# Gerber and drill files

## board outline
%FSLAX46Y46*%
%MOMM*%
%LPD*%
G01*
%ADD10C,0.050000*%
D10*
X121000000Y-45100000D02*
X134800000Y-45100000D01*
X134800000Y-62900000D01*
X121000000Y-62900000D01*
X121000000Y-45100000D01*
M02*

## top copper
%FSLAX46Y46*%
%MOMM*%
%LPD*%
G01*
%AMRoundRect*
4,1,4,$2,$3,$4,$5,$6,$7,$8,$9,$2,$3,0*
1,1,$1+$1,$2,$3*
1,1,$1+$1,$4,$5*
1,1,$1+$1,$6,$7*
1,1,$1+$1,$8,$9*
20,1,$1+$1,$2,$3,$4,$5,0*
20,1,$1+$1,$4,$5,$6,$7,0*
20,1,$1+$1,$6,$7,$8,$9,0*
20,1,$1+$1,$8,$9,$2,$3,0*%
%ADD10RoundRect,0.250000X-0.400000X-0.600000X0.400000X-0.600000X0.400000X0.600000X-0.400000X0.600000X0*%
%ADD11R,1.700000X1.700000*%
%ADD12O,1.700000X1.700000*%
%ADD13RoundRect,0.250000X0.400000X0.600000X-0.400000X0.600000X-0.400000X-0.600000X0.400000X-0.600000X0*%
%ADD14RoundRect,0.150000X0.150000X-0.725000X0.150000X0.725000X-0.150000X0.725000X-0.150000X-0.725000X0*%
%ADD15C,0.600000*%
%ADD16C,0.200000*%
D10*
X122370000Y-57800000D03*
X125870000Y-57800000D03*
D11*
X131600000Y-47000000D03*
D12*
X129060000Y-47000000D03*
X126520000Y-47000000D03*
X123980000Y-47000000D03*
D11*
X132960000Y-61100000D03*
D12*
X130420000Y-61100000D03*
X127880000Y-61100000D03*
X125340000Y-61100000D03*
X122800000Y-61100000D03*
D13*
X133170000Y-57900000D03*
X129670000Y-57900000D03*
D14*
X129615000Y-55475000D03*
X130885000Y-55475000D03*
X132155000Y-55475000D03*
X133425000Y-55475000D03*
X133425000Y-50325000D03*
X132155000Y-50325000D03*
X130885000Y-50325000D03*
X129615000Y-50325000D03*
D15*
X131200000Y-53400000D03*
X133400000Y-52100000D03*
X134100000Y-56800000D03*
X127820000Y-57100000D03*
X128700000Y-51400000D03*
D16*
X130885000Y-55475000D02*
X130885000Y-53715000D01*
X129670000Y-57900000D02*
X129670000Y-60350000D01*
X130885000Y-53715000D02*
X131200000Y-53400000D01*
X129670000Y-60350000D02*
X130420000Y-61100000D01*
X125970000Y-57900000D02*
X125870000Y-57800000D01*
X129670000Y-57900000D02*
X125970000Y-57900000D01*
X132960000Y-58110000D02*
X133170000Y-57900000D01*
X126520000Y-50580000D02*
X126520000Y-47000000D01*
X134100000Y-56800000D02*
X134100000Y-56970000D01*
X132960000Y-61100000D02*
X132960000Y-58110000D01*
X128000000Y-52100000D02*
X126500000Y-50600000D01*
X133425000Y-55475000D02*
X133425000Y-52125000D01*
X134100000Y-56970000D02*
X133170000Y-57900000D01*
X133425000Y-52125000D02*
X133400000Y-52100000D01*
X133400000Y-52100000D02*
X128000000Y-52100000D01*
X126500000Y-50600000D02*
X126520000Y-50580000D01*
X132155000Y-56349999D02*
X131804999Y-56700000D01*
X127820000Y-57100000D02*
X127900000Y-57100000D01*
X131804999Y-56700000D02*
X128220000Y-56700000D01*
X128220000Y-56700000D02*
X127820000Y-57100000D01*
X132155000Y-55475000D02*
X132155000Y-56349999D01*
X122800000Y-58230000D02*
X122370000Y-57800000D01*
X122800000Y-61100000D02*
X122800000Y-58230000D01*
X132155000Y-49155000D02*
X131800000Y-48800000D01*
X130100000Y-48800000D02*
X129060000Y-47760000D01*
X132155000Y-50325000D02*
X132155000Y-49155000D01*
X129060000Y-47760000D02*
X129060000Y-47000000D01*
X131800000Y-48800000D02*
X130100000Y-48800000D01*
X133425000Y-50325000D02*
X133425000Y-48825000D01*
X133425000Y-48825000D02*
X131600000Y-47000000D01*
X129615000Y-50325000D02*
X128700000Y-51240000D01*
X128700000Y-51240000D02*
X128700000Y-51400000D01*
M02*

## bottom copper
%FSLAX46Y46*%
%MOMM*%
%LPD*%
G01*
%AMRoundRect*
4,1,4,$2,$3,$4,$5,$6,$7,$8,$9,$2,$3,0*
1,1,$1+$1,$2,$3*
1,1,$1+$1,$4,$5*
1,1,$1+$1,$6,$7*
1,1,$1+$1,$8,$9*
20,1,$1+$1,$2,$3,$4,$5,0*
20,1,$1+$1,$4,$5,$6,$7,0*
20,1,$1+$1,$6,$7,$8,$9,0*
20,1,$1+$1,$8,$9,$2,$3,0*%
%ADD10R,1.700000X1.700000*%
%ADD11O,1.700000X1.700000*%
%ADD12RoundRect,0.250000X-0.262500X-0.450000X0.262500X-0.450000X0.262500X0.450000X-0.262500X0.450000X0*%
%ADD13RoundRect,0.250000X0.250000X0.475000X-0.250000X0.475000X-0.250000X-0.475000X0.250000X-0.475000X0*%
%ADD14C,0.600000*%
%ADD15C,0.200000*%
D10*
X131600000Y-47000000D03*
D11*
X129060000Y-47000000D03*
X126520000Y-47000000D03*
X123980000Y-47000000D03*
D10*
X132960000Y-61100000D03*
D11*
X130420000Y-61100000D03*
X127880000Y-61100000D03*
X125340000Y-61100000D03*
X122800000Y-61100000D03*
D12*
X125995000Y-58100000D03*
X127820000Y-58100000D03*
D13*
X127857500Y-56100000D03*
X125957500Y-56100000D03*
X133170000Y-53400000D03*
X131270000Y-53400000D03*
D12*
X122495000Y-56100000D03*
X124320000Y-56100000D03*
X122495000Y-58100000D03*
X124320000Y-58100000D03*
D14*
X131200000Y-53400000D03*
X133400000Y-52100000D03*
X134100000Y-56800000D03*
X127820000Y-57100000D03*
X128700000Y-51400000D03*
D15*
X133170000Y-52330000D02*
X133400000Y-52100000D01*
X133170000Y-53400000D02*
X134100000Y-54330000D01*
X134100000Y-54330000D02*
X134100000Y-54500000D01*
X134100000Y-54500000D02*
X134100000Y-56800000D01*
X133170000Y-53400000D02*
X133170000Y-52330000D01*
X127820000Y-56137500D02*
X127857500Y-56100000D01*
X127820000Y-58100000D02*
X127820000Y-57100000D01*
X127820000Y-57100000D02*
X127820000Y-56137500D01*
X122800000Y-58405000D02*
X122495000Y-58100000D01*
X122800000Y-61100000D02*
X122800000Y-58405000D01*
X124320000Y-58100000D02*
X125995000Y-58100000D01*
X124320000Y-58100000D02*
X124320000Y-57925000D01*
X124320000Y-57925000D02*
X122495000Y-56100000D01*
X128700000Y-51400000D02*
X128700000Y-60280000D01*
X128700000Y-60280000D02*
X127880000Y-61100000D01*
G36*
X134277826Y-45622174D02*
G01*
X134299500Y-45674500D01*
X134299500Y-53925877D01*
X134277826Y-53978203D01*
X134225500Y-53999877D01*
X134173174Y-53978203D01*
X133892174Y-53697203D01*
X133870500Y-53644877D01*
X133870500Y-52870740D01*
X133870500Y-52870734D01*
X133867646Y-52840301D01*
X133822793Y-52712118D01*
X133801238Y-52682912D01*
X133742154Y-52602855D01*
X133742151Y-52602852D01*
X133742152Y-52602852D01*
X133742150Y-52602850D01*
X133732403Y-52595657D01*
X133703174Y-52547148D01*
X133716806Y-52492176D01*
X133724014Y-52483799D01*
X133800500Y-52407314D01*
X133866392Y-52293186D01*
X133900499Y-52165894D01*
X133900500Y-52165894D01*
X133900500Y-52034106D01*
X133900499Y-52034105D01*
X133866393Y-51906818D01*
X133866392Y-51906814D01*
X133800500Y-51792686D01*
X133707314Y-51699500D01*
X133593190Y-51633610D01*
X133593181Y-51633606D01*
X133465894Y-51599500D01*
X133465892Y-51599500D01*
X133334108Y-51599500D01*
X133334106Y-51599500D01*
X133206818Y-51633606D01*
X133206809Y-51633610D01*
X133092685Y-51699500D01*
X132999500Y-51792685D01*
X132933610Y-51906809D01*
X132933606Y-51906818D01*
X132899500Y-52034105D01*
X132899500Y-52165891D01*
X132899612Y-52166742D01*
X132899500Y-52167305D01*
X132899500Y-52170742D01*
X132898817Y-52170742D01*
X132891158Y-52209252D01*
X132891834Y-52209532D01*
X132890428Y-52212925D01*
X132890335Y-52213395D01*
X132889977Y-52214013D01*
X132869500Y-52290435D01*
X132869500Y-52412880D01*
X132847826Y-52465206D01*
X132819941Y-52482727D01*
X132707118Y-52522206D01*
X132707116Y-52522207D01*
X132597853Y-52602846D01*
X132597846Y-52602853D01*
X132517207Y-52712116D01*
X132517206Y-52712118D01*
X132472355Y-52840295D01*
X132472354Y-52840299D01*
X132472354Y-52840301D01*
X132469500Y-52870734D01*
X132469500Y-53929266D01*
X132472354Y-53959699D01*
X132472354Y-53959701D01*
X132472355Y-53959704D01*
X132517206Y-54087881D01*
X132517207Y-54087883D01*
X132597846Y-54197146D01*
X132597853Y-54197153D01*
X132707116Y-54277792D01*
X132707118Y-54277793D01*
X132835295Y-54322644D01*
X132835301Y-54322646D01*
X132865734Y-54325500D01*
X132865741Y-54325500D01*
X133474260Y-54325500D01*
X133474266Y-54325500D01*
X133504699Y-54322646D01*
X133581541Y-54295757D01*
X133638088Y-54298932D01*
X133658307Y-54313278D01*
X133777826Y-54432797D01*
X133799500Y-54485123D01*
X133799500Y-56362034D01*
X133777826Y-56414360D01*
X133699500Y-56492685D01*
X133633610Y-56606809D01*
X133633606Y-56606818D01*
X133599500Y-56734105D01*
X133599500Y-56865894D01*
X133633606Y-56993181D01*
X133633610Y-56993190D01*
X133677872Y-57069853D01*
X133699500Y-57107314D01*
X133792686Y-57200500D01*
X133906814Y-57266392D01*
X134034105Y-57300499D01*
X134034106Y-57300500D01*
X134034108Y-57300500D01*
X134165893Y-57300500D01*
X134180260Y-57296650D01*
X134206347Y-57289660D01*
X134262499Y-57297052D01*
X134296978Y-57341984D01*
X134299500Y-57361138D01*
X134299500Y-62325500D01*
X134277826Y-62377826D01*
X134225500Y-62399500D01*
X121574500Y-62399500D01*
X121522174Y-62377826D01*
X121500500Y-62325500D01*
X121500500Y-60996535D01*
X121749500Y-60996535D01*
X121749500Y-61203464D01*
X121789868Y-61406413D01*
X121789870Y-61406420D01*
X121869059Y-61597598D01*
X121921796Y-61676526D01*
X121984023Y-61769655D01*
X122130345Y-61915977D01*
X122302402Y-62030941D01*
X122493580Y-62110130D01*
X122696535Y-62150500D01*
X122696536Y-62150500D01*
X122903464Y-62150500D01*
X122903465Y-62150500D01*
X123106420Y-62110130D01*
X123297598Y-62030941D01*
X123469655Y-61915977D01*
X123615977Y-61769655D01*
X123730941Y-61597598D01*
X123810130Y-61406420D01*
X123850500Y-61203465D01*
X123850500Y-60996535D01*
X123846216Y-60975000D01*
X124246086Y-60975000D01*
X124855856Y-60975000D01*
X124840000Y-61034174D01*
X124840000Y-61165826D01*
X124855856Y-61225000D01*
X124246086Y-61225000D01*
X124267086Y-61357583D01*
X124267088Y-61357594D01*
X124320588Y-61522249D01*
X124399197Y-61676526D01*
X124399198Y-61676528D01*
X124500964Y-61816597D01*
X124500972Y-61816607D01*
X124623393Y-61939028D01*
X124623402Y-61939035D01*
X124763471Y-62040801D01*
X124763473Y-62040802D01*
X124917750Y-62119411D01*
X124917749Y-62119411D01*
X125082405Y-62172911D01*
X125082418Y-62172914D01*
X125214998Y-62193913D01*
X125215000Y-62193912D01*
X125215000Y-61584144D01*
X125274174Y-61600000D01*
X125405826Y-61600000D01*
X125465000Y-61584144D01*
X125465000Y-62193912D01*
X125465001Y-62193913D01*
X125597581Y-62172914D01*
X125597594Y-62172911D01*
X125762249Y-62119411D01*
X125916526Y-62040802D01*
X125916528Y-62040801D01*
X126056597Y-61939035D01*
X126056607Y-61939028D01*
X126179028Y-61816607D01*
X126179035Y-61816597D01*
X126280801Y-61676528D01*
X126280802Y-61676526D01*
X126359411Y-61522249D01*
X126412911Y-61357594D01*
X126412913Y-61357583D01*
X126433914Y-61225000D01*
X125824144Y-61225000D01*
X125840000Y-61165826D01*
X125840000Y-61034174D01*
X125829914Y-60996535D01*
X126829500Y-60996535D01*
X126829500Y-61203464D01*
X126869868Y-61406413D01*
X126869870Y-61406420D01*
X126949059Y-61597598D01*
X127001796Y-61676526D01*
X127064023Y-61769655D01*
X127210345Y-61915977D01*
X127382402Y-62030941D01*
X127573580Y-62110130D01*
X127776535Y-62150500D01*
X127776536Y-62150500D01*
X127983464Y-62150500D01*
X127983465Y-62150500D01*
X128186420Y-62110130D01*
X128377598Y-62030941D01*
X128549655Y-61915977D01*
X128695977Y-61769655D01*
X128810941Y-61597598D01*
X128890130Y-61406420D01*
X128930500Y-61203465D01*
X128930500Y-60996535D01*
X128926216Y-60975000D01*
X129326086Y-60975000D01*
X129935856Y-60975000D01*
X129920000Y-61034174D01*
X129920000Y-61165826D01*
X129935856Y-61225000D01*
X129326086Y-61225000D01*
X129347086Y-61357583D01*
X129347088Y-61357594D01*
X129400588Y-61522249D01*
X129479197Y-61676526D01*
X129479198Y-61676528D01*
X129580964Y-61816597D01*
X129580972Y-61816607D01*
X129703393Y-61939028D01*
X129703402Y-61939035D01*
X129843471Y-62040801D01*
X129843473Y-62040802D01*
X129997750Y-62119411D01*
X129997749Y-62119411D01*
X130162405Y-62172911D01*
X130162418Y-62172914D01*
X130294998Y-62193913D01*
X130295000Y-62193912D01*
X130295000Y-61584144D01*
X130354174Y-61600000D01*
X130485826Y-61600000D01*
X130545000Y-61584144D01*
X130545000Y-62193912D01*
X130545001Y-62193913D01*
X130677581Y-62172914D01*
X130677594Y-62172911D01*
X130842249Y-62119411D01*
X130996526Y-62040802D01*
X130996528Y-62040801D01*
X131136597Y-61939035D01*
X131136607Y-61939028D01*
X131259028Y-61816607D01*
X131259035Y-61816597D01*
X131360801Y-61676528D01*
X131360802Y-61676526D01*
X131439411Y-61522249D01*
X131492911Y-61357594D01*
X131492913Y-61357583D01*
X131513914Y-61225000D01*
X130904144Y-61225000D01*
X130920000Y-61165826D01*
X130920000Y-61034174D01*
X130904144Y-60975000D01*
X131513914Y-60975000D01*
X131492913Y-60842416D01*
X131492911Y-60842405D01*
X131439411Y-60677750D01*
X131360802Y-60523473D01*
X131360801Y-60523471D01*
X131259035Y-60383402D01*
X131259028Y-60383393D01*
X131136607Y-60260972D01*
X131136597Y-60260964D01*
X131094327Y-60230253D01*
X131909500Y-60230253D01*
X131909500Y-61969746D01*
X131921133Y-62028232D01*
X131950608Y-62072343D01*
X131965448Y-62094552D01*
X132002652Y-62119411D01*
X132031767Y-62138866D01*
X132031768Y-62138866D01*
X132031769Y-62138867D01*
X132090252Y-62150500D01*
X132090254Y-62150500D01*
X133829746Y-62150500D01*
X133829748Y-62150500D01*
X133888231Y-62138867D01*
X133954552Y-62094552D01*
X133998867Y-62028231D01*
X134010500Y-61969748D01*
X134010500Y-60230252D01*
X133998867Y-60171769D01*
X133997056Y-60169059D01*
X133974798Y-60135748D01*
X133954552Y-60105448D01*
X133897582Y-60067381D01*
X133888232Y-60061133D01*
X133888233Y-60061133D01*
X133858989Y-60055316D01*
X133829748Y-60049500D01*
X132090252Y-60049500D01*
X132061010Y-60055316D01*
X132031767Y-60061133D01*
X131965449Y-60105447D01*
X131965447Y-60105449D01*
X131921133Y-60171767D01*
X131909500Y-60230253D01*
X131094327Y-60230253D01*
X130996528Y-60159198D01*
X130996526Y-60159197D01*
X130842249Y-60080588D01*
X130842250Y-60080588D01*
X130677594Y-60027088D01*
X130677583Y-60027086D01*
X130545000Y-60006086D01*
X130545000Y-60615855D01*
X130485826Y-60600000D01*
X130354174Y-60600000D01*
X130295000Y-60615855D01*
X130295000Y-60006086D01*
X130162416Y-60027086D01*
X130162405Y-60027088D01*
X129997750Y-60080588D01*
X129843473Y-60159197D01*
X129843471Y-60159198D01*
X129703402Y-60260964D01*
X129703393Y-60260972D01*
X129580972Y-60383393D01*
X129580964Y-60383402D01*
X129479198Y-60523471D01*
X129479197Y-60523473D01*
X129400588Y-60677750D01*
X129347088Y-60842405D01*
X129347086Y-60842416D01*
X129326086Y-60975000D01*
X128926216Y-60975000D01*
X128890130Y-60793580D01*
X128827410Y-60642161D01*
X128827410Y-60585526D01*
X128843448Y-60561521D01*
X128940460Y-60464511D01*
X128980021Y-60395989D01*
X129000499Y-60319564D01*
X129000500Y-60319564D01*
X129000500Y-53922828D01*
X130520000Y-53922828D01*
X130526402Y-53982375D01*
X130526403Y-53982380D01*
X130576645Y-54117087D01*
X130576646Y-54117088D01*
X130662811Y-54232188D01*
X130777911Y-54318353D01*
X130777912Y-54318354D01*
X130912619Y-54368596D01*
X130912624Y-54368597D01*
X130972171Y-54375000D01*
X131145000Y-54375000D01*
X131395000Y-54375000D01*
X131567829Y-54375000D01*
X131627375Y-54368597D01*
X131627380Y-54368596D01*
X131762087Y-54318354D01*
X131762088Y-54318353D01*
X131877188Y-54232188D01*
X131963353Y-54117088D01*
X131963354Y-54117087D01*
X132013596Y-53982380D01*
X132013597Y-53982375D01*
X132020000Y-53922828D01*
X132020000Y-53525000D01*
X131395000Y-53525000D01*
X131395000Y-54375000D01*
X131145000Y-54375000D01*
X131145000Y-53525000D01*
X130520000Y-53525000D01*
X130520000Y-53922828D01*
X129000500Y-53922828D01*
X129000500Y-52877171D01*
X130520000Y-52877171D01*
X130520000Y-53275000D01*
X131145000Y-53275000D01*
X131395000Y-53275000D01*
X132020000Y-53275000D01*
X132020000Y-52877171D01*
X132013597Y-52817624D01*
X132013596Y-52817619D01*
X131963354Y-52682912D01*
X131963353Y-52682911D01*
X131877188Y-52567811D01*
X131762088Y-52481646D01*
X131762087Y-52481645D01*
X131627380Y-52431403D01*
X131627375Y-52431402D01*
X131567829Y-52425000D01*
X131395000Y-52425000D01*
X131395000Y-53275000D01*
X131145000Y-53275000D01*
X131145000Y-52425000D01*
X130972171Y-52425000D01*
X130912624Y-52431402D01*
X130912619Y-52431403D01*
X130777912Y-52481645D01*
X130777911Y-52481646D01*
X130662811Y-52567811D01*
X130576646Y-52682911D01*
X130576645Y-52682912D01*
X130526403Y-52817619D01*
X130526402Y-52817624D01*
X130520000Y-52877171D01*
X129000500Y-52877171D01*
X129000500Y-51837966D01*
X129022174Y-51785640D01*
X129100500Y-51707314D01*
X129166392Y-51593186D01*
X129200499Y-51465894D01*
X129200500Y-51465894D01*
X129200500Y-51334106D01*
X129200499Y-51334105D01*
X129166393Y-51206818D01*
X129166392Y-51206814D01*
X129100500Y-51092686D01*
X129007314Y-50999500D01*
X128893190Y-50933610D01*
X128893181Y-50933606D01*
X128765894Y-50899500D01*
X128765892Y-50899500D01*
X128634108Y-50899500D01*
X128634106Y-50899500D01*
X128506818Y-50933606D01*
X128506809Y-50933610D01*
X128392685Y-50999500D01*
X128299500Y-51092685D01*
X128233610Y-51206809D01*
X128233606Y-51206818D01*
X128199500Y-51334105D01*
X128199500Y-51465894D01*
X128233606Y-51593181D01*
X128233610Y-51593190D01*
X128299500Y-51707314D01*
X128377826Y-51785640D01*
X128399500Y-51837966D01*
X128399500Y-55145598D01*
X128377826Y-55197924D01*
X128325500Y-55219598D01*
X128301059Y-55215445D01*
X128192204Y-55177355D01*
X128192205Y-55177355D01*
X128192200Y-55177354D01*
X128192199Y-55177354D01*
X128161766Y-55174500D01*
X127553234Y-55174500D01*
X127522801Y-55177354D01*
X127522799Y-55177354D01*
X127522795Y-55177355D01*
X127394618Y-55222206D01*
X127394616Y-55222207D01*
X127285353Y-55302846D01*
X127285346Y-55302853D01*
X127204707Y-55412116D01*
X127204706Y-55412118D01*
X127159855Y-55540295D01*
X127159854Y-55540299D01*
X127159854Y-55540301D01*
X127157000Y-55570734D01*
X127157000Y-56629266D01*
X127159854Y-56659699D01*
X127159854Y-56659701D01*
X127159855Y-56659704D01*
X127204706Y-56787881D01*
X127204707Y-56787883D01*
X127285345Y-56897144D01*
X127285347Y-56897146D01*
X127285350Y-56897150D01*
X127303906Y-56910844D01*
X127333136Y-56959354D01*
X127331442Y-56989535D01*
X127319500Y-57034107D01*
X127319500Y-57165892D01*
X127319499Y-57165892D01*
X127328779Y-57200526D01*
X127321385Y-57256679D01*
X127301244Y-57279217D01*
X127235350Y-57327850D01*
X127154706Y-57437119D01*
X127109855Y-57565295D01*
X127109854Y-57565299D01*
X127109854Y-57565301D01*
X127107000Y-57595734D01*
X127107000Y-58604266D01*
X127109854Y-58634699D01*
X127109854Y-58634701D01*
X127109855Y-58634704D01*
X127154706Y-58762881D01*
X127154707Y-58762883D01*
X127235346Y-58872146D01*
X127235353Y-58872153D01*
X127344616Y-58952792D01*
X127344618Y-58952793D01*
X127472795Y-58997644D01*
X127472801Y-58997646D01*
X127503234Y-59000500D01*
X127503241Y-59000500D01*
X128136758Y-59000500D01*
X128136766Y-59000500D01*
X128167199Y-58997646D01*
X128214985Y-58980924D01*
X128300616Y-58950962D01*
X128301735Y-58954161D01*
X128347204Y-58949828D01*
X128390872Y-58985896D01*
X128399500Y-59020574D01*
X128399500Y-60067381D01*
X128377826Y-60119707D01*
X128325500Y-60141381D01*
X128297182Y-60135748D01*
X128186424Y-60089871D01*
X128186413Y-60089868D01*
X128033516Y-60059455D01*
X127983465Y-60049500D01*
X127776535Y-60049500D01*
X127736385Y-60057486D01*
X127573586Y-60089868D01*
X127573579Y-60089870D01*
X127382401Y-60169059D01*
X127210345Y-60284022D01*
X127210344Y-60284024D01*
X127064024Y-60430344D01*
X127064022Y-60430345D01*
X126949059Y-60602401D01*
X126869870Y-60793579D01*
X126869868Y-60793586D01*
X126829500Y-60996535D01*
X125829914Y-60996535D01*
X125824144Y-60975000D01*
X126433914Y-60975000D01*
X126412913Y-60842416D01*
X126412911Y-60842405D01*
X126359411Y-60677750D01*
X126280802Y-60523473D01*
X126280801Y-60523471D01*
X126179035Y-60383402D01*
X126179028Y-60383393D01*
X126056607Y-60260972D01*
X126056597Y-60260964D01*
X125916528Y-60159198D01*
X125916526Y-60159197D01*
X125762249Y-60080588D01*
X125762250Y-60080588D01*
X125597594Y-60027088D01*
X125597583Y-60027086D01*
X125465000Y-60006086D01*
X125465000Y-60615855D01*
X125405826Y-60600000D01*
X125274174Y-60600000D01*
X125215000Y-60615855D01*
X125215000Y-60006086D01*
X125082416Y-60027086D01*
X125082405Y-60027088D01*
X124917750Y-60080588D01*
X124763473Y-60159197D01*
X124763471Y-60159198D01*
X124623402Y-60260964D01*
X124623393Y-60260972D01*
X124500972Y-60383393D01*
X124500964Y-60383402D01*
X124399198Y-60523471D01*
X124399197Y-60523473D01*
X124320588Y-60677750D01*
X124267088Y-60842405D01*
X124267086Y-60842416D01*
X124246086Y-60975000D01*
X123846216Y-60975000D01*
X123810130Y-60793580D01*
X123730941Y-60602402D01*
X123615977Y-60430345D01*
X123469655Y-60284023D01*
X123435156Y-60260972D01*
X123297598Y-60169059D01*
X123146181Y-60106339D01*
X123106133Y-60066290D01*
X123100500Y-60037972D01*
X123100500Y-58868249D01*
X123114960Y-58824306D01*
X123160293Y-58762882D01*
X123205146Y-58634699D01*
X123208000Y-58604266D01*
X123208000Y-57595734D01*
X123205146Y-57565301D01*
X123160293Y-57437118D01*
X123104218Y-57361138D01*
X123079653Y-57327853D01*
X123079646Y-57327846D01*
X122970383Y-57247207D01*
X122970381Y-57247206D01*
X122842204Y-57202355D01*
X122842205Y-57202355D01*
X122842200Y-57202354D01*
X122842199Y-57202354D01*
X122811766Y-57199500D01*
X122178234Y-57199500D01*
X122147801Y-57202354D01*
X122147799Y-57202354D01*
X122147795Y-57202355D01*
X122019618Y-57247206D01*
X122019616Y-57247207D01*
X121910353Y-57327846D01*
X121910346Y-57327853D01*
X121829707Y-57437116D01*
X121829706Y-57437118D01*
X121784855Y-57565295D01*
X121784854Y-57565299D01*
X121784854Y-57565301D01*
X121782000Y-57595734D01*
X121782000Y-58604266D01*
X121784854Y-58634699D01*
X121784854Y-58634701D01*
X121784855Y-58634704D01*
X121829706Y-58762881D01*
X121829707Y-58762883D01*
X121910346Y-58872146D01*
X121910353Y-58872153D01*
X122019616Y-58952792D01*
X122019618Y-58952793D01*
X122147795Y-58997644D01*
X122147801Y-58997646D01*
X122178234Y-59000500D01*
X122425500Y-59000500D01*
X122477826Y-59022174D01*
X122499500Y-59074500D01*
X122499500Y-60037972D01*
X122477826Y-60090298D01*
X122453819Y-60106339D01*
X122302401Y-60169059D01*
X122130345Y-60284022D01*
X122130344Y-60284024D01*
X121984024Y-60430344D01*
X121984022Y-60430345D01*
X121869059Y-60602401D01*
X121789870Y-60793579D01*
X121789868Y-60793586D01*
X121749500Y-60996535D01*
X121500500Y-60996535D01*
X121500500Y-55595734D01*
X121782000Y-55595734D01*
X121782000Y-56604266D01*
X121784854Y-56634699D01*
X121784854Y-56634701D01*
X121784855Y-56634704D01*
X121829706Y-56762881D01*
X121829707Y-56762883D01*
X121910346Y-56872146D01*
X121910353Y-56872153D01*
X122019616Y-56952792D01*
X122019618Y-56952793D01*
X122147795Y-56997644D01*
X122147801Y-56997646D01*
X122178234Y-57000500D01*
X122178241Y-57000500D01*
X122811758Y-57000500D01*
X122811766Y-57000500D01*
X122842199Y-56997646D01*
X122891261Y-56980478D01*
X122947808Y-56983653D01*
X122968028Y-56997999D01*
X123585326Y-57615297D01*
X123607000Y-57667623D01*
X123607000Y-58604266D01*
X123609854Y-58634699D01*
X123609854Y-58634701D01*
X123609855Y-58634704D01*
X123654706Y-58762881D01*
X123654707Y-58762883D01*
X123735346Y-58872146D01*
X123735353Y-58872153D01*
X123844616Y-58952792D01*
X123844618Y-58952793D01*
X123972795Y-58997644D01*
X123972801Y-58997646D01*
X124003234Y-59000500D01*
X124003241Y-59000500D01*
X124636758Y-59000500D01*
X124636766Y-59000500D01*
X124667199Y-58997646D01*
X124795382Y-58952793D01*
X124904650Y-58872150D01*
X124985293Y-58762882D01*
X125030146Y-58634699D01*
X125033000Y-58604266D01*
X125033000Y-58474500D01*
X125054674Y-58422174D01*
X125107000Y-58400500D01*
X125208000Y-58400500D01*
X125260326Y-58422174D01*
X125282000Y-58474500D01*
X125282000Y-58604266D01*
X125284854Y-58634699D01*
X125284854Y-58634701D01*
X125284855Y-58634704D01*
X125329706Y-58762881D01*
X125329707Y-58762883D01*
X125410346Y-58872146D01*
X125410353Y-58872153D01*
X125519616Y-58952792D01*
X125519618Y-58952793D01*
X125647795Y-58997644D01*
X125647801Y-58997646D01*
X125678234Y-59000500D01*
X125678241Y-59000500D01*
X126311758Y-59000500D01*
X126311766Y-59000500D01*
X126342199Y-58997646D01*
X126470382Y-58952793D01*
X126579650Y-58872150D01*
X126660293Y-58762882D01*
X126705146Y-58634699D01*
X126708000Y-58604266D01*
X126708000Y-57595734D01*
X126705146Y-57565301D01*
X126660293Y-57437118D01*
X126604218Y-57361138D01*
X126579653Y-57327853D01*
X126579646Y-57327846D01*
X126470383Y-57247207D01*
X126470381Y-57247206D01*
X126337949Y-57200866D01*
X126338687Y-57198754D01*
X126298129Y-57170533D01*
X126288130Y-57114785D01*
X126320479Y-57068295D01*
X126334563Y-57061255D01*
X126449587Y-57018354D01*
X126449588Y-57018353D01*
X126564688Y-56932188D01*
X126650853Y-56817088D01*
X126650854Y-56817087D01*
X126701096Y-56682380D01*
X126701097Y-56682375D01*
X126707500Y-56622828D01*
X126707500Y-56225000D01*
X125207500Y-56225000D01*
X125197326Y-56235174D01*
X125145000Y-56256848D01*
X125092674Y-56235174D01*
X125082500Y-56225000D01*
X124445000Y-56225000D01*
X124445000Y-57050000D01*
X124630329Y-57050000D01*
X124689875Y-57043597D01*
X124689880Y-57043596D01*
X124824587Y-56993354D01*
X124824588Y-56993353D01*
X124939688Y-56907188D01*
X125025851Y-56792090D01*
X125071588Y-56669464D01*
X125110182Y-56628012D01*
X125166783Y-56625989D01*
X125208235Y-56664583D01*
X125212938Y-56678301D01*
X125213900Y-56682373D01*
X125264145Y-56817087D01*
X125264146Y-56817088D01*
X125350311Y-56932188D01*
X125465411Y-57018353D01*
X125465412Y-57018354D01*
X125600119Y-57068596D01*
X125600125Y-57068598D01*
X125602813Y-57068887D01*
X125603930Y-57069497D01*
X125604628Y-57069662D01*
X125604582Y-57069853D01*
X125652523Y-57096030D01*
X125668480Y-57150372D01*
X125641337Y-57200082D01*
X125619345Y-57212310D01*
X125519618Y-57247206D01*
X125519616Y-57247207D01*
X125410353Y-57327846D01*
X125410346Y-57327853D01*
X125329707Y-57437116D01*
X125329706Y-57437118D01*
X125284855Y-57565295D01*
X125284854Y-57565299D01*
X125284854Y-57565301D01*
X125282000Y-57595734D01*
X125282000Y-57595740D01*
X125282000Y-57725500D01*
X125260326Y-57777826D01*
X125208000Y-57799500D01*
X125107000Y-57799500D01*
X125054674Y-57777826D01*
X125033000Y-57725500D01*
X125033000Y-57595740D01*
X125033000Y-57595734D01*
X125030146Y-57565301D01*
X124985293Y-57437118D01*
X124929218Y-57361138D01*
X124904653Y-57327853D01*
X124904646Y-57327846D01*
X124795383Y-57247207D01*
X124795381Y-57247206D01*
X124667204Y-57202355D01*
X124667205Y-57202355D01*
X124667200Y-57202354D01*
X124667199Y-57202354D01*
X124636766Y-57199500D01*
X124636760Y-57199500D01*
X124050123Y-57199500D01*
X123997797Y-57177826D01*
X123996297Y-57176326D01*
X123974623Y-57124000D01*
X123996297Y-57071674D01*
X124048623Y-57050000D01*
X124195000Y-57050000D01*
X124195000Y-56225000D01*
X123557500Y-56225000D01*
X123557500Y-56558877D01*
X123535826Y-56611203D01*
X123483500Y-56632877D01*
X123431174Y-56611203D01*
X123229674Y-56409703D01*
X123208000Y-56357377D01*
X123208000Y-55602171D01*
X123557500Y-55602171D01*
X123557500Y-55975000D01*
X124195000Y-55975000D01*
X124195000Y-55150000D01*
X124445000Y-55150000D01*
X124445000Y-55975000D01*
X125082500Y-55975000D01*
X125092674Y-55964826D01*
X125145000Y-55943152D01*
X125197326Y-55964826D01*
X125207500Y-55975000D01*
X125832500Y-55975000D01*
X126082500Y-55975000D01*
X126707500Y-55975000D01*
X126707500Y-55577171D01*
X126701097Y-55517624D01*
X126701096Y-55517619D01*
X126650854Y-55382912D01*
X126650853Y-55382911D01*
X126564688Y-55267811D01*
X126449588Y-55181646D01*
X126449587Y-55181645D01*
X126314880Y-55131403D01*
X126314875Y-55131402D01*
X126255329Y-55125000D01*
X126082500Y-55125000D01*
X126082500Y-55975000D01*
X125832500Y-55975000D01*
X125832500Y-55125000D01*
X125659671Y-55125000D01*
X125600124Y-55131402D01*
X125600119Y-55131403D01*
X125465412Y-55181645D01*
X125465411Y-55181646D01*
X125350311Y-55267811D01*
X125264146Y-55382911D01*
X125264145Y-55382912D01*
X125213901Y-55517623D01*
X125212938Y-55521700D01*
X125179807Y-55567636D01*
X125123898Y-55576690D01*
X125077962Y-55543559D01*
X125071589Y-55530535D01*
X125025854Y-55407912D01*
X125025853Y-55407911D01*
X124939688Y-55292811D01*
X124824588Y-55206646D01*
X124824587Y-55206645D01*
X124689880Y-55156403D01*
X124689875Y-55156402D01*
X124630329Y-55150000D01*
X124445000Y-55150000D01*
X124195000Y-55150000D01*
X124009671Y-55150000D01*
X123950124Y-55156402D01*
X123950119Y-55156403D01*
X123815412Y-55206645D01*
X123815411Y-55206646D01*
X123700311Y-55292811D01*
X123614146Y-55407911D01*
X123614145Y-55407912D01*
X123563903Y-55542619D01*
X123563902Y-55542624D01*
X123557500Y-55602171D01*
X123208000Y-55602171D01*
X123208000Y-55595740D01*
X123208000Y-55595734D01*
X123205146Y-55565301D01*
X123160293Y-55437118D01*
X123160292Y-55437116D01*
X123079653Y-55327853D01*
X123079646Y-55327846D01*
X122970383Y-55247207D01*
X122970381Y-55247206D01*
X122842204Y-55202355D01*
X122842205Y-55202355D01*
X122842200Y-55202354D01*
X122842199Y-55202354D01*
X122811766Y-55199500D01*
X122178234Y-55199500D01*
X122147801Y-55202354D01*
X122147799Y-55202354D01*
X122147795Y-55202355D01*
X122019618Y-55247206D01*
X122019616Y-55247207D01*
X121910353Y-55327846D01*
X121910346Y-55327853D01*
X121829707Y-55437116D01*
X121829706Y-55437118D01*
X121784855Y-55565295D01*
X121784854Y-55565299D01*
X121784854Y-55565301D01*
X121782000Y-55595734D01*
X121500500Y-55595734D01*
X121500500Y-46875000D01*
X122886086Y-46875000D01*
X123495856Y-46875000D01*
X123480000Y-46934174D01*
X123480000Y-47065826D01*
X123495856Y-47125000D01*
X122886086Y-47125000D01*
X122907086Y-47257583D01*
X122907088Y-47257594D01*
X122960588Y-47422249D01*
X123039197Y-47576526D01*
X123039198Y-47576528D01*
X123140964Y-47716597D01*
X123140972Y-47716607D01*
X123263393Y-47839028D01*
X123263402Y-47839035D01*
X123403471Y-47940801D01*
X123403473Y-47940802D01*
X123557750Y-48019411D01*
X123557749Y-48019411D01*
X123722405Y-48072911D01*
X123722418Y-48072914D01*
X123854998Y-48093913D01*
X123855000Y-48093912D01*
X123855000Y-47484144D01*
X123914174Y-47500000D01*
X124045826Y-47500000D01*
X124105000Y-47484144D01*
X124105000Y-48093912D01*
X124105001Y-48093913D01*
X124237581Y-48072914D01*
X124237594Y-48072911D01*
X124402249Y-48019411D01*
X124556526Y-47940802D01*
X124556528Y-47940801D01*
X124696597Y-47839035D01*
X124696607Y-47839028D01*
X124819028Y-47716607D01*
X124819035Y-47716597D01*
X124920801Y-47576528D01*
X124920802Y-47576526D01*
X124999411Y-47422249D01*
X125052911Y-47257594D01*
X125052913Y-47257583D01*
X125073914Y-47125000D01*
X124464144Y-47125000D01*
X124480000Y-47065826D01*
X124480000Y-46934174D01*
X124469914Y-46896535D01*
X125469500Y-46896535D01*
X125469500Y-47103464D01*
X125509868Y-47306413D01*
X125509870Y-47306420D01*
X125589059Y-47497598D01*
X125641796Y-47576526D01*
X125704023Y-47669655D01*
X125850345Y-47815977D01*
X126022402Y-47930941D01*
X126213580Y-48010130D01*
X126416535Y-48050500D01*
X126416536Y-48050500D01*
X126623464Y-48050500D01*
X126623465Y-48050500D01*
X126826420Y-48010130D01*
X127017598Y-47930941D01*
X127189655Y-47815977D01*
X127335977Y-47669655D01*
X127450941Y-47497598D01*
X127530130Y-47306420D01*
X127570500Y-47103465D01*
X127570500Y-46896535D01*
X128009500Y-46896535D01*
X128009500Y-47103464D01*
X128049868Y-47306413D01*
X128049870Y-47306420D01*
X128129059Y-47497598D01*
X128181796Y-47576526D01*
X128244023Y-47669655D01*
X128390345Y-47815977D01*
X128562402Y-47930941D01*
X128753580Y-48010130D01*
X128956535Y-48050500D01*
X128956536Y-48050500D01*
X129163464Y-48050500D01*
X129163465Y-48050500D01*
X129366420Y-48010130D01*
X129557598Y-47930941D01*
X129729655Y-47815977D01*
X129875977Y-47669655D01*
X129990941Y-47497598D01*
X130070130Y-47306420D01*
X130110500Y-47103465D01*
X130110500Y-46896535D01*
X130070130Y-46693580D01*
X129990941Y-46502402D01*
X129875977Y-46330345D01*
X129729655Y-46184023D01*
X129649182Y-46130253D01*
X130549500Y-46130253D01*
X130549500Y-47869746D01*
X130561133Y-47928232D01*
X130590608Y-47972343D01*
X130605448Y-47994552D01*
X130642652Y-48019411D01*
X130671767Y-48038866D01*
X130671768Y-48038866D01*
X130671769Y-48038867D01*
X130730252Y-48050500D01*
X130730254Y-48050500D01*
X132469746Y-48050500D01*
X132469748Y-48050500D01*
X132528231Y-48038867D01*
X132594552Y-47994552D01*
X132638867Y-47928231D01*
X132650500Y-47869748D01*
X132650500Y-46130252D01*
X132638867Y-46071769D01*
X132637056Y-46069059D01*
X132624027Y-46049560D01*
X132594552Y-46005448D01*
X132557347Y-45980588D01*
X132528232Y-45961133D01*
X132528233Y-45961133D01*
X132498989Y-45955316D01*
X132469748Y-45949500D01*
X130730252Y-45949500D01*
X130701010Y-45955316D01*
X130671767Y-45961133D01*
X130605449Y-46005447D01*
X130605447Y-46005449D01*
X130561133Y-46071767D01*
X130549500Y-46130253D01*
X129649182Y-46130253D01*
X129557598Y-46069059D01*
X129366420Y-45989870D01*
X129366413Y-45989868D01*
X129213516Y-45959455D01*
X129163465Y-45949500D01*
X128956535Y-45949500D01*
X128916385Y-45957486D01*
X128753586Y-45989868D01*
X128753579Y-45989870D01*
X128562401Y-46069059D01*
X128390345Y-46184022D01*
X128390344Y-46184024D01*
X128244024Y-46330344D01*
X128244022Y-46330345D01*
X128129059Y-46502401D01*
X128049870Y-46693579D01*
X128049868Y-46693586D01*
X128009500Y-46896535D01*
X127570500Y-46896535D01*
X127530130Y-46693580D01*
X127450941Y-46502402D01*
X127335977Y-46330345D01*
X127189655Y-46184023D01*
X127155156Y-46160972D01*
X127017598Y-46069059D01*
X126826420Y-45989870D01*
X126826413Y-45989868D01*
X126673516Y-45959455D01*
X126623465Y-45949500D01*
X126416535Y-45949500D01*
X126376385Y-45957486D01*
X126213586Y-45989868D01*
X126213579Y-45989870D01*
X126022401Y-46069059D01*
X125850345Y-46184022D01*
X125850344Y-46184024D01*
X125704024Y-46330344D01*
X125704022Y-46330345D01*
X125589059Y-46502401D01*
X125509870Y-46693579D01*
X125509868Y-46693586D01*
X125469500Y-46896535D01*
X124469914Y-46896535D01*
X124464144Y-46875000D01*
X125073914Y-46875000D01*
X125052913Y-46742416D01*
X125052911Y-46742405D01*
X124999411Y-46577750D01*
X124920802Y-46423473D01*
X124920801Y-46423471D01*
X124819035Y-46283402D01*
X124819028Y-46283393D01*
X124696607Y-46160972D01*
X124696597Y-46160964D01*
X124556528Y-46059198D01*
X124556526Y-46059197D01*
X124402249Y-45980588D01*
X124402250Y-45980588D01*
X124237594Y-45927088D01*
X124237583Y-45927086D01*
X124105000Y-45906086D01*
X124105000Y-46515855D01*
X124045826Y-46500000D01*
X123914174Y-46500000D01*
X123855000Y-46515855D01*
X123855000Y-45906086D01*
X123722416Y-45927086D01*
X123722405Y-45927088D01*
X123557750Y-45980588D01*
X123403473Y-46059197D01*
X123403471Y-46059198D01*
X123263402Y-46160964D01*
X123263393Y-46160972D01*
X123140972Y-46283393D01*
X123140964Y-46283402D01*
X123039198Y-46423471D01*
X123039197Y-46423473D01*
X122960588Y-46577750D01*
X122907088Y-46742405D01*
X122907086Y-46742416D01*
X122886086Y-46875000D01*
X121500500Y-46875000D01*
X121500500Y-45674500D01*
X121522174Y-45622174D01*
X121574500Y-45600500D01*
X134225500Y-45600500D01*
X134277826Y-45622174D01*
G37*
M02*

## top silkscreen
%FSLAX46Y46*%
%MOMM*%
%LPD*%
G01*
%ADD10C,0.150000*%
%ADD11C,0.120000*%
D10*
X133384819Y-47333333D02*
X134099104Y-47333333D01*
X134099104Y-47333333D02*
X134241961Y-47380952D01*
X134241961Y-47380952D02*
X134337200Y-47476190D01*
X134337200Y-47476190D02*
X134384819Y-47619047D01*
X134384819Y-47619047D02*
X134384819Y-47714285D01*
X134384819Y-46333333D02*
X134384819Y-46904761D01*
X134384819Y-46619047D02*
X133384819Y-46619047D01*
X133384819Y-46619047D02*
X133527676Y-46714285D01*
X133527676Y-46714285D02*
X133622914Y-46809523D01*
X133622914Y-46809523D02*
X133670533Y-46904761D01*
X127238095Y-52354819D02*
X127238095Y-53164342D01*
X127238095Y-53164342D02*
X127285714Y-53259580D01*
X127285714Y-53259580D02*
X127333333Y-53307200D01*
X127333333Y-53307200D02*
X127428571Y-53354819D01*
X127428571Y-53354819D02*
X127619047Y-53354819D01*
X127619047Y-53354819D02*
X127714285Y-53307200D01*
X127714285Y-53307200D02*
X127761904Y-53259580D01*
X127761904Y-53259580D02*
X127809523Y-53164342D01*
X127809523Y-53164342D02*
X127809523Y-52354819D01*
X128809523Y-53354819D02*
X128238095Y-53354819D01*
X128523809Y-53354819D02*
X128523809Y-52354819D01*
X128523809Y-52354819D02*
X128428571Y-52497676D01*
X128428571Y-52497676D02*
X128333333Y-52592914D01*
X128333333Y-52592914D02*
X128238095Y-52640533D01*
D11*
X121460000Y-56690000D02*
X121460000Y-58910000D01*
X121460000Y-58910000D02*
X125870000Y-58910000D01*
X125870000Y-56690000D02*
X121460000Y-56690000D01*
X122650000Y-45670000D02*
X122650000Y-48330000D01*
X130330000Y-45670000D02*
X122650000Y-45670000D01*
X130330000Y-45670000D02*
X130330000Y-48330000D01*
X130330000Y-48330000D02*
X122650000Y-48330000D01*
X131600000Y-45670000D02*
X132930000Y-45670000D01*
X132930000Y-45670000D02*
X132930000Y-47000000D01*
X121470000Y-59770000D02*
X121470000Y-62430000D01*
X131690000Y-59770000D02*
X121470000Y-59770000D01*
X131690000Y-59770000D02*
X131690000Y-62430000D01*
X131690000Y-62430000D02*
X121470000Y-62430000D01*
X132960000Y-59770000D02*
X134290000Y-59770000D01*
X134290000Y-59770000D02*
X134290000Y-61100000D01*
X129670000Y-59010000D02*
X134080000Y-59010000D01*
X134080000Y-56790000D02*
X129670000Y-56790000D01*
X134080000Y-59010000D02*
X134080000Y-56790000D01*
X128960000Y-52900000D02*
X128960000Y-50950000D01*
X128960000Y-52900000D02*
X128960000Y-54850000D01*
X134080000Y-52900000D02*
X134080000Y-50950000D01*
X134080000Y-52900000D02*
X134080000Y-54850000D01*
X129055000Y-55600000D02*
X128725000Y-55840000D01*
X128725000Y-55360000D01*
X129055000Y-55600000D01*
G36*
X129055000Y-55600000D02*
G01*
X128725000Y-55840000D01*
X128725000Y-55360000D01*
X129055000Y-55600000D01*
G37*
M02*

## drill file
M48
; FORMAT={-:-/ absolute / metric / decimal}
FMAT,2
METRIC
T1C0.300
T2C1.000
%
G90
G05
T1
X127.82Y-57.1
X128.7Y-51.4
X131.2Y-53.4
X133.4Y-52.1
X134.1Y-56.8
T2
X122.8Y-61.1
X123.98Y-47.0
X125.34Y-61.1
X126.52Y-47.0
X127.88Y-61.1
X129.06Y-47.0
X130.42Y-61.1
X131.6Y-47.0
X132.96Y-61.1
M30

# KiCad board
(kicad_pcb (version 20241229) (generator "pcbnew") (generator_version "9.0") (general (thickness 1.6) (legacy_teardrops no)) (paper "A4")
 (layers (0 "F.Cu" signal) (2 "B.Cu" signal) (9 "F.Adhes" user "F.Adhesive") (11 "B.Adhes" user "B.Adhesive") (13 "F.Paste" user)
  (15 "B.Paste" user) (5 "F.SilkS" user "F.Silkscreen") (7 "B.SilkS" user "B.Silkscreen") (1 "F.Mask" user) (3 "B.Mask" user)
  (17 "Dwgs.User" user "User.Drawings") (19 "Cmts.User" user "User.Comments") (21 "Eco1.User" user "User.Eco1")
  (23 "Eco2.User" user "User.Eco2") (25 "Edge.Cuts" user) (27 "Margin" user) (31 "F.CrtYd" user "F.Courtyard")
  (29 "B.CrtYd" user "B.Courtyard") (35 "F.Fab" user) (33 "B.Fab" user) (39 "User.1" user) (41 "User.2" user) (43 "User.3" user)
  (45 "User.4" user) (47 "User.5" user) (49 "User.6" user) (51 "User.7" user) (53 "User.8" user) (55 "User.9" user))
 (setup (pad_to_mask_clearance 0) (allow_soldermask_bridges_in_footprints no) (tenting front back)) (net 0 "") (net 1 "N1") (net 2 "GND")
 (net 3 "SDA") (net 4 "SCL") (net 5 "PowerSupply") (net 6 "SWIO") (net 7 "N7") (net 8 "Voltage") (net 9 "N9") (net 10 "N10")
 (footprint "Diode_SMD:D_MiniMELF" (layer "F.Cu") (at 124.12 57.8)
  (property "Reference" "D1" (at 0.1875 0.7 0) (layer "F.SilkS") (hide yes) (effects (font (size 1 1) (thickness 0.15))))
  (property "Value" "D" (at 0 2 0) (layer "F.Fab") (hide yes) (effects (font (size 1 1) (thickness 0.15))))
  (fp_line (start -2.66 -1.11) (end -2.66 1.11) (stroke (width 0.12) (type solid)) (layer "F.SilkS"))
  (fp_line (start -2.66 1.11) (end 1.75 1.11) (stroke (width 0.12) (type solid)) (layer "F.SilkS"))
  (fp_line (start 1.75 -1.11) (end -2.66 -1.11) (stroke (width 0.12) (type solid)) (layer "F.SilkS"))
  (pad "1" smd roundrect (at -1.75 0) (size 1.3 1.7) (layers "F.Cu" "F.Mask" "F.Paste") (roundrect_rratio 0.1923076923) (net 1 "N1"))
  (pad "2" smd roundrect (at 1.75 0) (size 1.3 1.7) (layers "F.Cu" "F.Mask" "F.Paste") (roundrect_rratio 0.1923076923) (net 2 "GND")))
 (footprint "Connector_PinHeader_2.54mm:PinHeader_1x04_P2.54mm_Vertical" (layer "F.Cu") (at 131.6 47 -90)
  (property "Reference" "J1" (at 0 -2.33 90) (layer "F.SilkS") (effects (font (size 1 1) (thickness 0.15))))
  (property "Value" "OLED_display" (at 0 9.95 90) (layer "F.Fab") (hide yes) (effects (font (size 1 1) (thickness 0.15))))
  (fp_line (start -1.33 8.95) (end 1.33 8.95) (stroke (width 0.12) (type solid)) (layer "F.SilkS"))
  (fp_line (start -1.33 1.27) (end -1.33 8.95) (stroke (width 0.12) (type solid)) (layer "F.SilkS"))
  (fp_line (start -1.33 1.27) (end 1.33 1.27) (stroke (width 0.12) (type solid)) (layer "F.SilkS"))
  (fp_line (start 1.33 1.27) (end 1.33 8.95) (stroke (width 0.12) (type solid)) (layer "F.SilkS"))
  (fp_line (start -1.33 0) (end -1.33 -1.33) (stroke (width 0.12) (type solid)) (layer "F.SilkS"))
  (fp_line (start -1.33 -1.33) (end 0 -1.33) (stroke (width 0.12) (type solid)) (layer "F.SilkS"))
  (pad "1" thru_hole rect (at 0 0 270) (size 1.7 1.7) (drill 1) (layers "*.Cu" "*.Mask") (remove_unused_layers no) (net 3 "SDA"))
  (pad "2" thru_hole oval (at 0 2.54 270) (size 1.7 1.7) (drill 1) (layers "*.Cu" "*.Mask") (remove_unused_layers no) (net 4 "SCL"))
  (pad "3" thru_hole oval (at 0 5.08 270) (size 1.7 1.7) (drill 1) (layers "*.Cu" "*.Mask") (remove_unused_layers no) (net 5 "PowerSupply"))
  (pad "4" thru_hole oval (at 0 7.62 270) (size 1.7 1.7) (drill 1) (layers "*.Cu" "*.Mask") (remove_unused_layers no) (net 2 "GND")))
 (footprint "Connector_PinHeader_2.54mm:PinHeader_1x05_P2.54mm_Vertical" (layer "F.Cu") (at 132.96 61.1 -90)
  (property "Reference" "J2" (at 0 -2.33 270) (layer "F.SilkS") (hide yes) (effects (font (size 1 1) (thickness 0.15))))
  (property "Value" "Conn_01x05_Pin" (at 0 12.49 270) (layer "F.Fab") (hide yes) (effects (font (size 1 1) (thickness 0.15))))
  (fp_line (start -1.33 11.49) (end 1.33 11.49) (stroke (width 0.12) (type solid)) (layer "F.SilkS"))
  (fp_line (start -1.33 1.27) (end -1.33 11.49) (stroke (width 0.12) (type solid)) (layer "F.SilkS"))
  (fp_line (start -1.33 1.27) (end 1.33 1.27) (stroke (width 0.12) (type solid)) (layer "F.SilkS"))
  (fp_line (start 1.33 1.27) (end 1.33 11.49) (stroke (width 0.12) (type solid)) (layer "F.SilkS"))
  (fp_line (start -1.33 0) (end -1.33 -1.33) (stroke (width 0.12) (type solid)) (layer "F.SilkS"))
  (fp_line (start -1.33 -1.33) (end 0 -1.33) (stroke (width 0.12) (type solid)) (layer "F.SilkS"))
  (pad "1" thru_hole rect (at 0 0 270) (size 1.7 1.7) (drill 1) (layers "*.Cu" "*.Mask") (remove_unused_layers no) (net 5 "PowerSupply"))
  (pad "2" thru_hole oval (at 0 2.54 270) (size 1.7 1.7) (drill 1) (layers "*.Cu" "*.Mask") (remove_unused_layers no) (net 2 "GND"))
  (pad "3" thru_hole oval (at 0 5.08 270) (size 1.7 1.7) (drill 1) (layers "*.Cu" "*.Mask") (remove_unused_layers no) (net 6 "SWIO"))
  (pad "4" thru_hole oval (at 0 7.62 270) (size 1.7 1.7) (drill 1) (layers "*.Cu" "*.Mask") (remove_unused_layers no) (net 2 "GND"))
  (pad "5" thru_hole oval (at 0 10.16 270) (size 1.7 1.7) (drill 1) (layers "*.Cu" "*.Mask") (remove_unused_layers no) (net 1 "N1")))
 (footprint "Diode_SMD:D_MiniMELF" (layer "F.Cu") (at 131.42 57.9 180)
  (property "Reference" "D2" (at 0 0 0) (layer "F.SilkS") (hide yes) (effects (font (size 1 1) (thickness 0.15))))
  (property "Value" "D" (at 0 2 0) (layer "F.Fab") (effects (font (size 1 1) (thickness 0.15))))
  (fp_line (start 1.75 -1.11) (end -2.66 -1.11) (stroke (width 0.12) (type solid)) (layer "F.SilkS"))
  (fp_line (start -2.66 1.11) (end 1.75 1.11) (stroke (width 0.12) (type solid)) (layer "F.SilkS"))
  (fp_line (start -2.66 -1.11) (end -2.66 1.11) (stroke (width 0.12) (type solid)) (layer "F.SilkS"))
  (pad "1" smd roundrect (at -1.75 0 180) (size 1.3 1.7) (layers "F.Cu" "F.Mask" "F.Paste") (roundrect_rratio 0.1923076923)
   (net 5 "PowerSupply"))
  (pad "2" smd roundrect (at 1.75 0 180) (size 1.3 1.7) (layers "F.Cu" "F.Mask" "F.Paste") (roundrect_rratio 0.1923076923) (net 2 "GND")))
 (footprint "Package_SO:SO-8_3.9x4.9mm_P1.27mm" (layer "F.Cu") (at 131.52 52.9 90)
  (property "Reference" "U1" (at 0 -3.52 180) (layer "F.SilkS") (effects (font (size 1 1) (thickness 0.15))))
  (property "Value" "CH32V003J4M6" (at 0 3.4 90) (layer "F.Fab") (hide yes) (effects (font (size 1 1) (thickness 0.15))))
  (fp_line (start 0 -2.56) (end 1.95 -2.56) (stroke (width 0.12) (type solid)) (layer "F.SilkS"))
  (fp_line (start 0 -2.56) (end -1.95 -2.56) (stroke (width 0.12) (type solid)) (layer "F.SilkS"))
  (fp_line (start 0 2.56) (end 1.95 2.56) (stroke (width 0.12) (type solid)) (layer "F.SilkS"))
  (fp_line (start 0 2.56) (end -1.95 2.56) (stroke (width 0.12) (type solid)) (layer "F.SilkS"))
  (fp_poly
   (pts (xy -2.7 -2.465) (xy -2.94 -2.795) (xy -2.46 -2.795) (xy -2.7 -2.465)) (stroke (width 0.12) (type solid)) (fill yes)
   (layer "F.SilkS"))
  (pad "1" smd roundrect (at -2.575 -1.905 90) (size 1.75 0.6) (layers "F.Cu" "F.Mask" "F.Paste") (roundrect_rratio 0.25) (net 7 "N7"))
  (pad "2" smd roundrect (at -2.575 -0.635 90) (size 1.75 0.6) (layers "F.Cu" "F.Mask" "F.Paste") (roundrect_rratio 0.25) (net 2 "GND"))
  (pad "3" smd roundrect (at -2.575 0.635 90) (size 1.75 0.6) (layers "F.Cu" "F.Mask" "F.Paste") (roundrect_rratio 0.25) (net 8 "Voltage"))
  (pad "4" smd roundrect (at -2.575 1.905 90) (size 1.75 0.6) (layers "F.Cu" "F.Mask" "F.Paste") (roundrect_rratio 0.25)
   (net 5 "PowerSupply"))
  (pad "5" smd roundrect (at 2.575 1.905 90) (size 1.75 0.6) (layers "F.Cu" "F.Mask" "F.Paste") (roundrect_rratio 0.25) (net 3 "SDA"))
  (pad "6" smd roundrect (at 2.575 0.635 90) (size 1.75 0.6) (layers "F.Cu" "F.Mask" "F.Paste") (roundrect_rratio 0.25) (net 4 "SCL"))
  (pad "7" smd roundrect (at 2.575 -0.635 90) (size 1.75 0.6) (layers "F.Cu" "F.Mask" "F.Paste") (roundrect_rratio 0.25) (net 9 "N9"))
  (pad "8" smd roundrect (at 2.575 -1.905 90) (size 1.75 0.6) (layers "F.Cu" "F.Mask" "F.Paste") (roundrect_rratio 0.25) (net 6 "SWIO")))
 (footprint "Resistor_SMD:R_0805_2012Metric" (layer "B.Cu") (at 126.9075 58.1)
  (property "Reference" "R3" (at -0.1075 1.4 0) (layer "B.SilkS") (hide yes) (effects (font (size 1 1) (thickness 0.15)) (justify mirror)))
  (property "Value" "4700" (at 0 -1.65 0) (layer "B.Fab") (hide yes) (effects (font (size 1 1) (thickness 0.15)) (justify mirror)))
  (pad "1" smd roundrect (at -0.9125 0) (size 1.025 1.4) (layers "B.Cu" "B.Mask" "B.Paste") (roundrect_rratio 0.243902) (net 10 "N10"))
  (pad "2" smd roundrect (at 0.9125 0) (size 1.025 1.4) (layers "B.Cu" "B.Mask" "B.Paste") (roundrect_rratio 0.243902) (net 8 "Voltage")))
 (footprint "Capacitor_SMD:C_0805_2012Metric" (layer "B.Cu") (at 126.9075 56.1 180)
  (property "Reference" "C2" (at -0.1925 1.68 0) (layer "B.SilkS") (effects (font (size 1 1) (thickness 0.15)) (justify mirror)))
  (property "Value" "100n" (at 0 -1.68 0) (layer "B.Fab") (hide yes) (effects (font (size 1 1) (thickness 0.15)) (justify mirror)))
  (pad "1" smd roundrect (at -0.95 0 180) (size 1 1.45) (layers "B.Cu" "B.Mask" "B.Paste") (roundrect_rratio 0.25) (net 8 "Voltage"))
  (pad "2" smd roundrect (at 0.95 0 180) (size 1 1.45) (layers "B.Cu" "B.Mask" "B.Paste") (roundrect_rratio 0.25) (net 2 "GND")))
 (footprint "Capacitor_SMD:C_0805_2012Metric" (layer "B.Cu") (at 132.22 53.4 180)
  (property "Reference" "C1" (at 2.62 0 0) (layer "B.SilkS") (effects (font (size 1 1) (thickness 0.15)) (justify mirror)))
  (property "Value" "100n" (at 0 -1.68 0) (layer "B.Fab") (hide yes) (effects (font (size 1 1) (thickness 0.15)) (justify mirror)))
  (pad "1" smd roundrect (at -0.95 0 180) (size 1 1.45) (layers "B.Cu" "B.Mask" "B.Paste") (roundrect_rratio 0.25) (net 5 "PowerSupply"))
  (pad "2" smd roundrect (at 0.95 0 180) (size 1 1.45) (layers "B.Cu" "B.Mask" "B.Paste") (roundrect_rratio 0.25) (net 2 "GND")))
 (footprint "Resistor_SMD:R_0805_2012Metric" (layer "B.Cu") (at 123.4075 56.1)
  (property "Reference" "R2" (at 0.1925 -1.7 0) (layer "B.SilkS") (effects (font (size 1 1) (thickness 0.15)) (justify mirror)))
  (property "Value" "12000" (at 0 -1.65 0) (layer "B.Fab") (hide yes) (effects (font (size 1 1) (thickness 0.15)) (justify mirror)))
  (pad "1" smd roundrect (at -0.9125 0) (size 1.025 1.4) (layers "B.Cu" "B.Mask" "B.Paste") (roundrect_rratio 0.243902) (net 10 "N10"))
  (pad "2" smd roundrect (at 0.9125 0) (size 1.025 1.4) (layers "B.Cu" "B.Mask" "B.Paste") (roundrect_rratio 0.243902) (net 2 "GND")))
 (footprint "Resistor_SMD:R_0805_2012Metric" (layer "B.Cu") (at 123.4075 58.1)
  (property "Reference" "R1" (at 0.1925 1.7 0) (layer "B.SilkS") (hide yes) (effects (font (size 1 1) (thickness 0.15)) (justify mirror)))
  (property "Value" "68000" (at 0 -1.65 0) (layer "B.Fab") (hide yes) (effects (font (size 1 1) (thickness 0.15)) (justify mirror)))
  (pad "1" smd roundrect (at -0.9125 0) (size 1.025 1.4) (layers "B.Cu" "B.Mask" "B.Paste") (roundrect_rratio 0.243902) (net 1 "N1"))
  (pad "2" smd roundrect (at 0.9125 0) (size 1.025 1.4) (layers "B.Cu" "B.Mask" "B.Paste") (roundrect_rratio 0.243902) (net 10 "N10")))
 (gr_rect (start 121 45.1) (end 134.8 62.9) (stroke (width 0.05) (type default)) (fill no) (layer "Edge.Cuts"))
 (segment (start 130.885 55.475) (end 130.885 53.715) (width 0.2) (layer "F.Cu") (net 2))
 (segment (start 129.67 57.9) (end 129.67 60.35) (width 0.2) (layer "F.Cu") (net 2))
 (segment (start 130.885 53.715) (end 131.2 53.4) (width 0.2) (layer "F.Cu") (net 2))
 (segment (start 129.67 60.35) (end 130.42 61.1) (width 0.2) (layer "F.Cu") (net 2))
 (segment (start 125.97 57.9) (end 125.87 57.8) (width 0.2) (layer "F.Cu") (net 2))
 (segment (start 129.67 57.9) (end 125.97 57.9) (width 0.2) (layer "F.Cu") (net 2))
 (via (at 131.2 53.4) (size 0.6) (drill 0.3) (layers "F.Cu" "B.Cu") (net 2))
 (segment (start 132.96 58.11) (end 133.17 57.9) (width 0.2) (layer "F.Cu") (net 5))
 (segment (start 126.52 50.58) (end 126.52 47) (width 0.2) (layer "F.Cu") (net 5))
 (segment (start 134.1 56.8) (end 134.1 56.97) (width 0.2) (layer "F.Cu") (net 5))
 (segment (start 132.96 61.1) (end 132.96 58.11) (width 0.2) (layer "F.Cu") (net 5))
 (segment (start 128 52.1) (end 126.5 50.6) (width 0.2) (layer "F.Cu") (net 5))
 (segment (start 133.425 55.475) (end 133.425 52.125) (width 0.2) (layer "F.Cu") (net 5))
 (segment (start 134.1 56.97) (end 133.17 57.9) (width 0.2) (layer "F.Cu") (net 5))
 (segment (start 133.425 52.125) (end 133.4 52.1) (width 0.2) (layer "F.Cu") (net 5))
 (segment (start 133.4 52.1) (end 128 52.1) (width 0.2) (layer "F.Cu") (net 5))
 (segment (start 126.5 50.6) (end 126.52 50.58) (width 0.2) (layer "F.Cu") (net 5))
 (via (at 133.4 52.1) (size 0.6) (drill 0.3) (layers "F.Cu" "B.Cu") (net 5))
 (via (at 134.1 56.8) (size 0.6) (drill 0.3) (layers "F.Cu" "B.Cu") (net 5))
 (segment (start 133.17 52.33) (end 133.4 52.1) (width 0.2) (layer "B.Cu") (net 5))
 (segment (start 133.17 53.4) (end 134.1 54.33) (width 0.2) (layer "B.Cu") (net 5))
 (segment (start 134.1 54.33) (end 134.1 54.5) (width 0.2) (layer "B.Cu") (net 5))
 (segment (start 134.1 54.5) (end 134.1 56.8) (width 0.2) (layer "B.Cu") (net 5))
 (segment (start 133.17 53.4) (end 133.17 52.33) (width 0.2) (layer "B.Cu") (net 5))
 (segment (start 132.155 56.349999) (end 131.804999 56.7) (width 0.2) (layer "F.Cu") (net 8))
 (segment (start 127.82 57.1) (end 127.9 57.1) (width 0.2) (layer "F.Cu") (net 8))
 (segment (start 131.804999 56.7) (end 128.22 56.7) (width 0.2) (layer "F.Cu") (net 8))
 (segment (start 128.22 56.7) (end 127.82 57.1) (width 0.2) (layer "F.Cu") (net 8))
 (segment (start 132.155 55.475) (end 132.155 56.349999) (width 0.2) (layer "F.Cu") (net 8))
 (via (at 127.82 57.1) (size 0.6) (drill 0.3) (layers "F.Cu" "B.Cu") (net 8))
 (segment (start 127.82 56.1375) (end 127.8575 56.1) (width 0.2) (layer "B.Cu") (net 8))
 (segment (start 127.82 58.1) (end 127.82 57.1) (width 0.2) (layer "B.Cu") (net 8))
 (segment (start 127.82 57.1) (end 127.82 56.1375) (width 0.2) (layer "B.Cu") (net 8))
 (segment (start 122.8 58.23) (end 122.37 57.8) (width 0.2) (layer "F.Cu") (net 1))
 (segment (start 122.8 61.1) (end 122.8 58.23) (width 0.2) (layer "F.Cu") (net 1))
 (segment (start 122.8 58.405) (end 122.495 58.1) (width 0.2) (layer "B.Cu") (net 1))
 (segment (start 122.8 61.1) (end 122.8 58.405) (width 0.2) (layer "B.Cu") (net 1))
 (segment (start 132.155 49.155) (end 131.8 48.8) (width 0.2) (layer "F.Cu") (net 4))
 (segment (start 130.1 48.8) (end 129.06 47.76) (width 0.2) (layer "F.Cu") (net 4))
 (segment (start 132.155 50.325) (end 132.155 49.155) (width 0.2) (layer "F.Cu") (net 4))
 (segment (start 129.06 47.76) (end 129.06 47) (width 0.2) (layer "F.Cu") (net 4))
 (segment (start 131.8 48.8) (end 130.1 48.8) (width 0.2) (layer "F.Cu") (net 4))
 (segment (start 133.425 50.325) (end 133.425 48.825) (width 0.2) (layer "F.Cu") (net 3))
 (segment (start 133.425 48.825) (end 131.6 47) (width 0.2) (layer "F.Cu") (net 3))
 (segment (start 124.32 58.1) (end 125.995 58.1) (width 0.2) (layer "B.Cu") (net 10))
 (segment (start 124.32 58.1) (end 124.32 57.925) (width 0.2) (layer "B.Cu") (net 10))
 (segment (start 124.32 57.925) (end 122.495 56.1) (width 0.2) (layer "B.Cu") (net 10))
 (segment (start 129.615 50.325) (end 128.7 51.24) (width 0.2) (layer "F.Cu") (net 6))
 (segment (start 128.7 51.24) (end 128.7 51.4) (width 0.2) (layer "F.Cu") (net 6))
 (via (at 128.7 51.4) (size 0.6) (drill 0.3) (layers "F.Cu" "B.Cu") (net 6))
 (segment (start 128.7 51.4) (end 128.7 60.28) (width 0.2) (layer "B.Cu") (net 6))
 (segment (start 128.7 60.28) (end 127.88 61.1) (width 0.2) (layer "B.Cu") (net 6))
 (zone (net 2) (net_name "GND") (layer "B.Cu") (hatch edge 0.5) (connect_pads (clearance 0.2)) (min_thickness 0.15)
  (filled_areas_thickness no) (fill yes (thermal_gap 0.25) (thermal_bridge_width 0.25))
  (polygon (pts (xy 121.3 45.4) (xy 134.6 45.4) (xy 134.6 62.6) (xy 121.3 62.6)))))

